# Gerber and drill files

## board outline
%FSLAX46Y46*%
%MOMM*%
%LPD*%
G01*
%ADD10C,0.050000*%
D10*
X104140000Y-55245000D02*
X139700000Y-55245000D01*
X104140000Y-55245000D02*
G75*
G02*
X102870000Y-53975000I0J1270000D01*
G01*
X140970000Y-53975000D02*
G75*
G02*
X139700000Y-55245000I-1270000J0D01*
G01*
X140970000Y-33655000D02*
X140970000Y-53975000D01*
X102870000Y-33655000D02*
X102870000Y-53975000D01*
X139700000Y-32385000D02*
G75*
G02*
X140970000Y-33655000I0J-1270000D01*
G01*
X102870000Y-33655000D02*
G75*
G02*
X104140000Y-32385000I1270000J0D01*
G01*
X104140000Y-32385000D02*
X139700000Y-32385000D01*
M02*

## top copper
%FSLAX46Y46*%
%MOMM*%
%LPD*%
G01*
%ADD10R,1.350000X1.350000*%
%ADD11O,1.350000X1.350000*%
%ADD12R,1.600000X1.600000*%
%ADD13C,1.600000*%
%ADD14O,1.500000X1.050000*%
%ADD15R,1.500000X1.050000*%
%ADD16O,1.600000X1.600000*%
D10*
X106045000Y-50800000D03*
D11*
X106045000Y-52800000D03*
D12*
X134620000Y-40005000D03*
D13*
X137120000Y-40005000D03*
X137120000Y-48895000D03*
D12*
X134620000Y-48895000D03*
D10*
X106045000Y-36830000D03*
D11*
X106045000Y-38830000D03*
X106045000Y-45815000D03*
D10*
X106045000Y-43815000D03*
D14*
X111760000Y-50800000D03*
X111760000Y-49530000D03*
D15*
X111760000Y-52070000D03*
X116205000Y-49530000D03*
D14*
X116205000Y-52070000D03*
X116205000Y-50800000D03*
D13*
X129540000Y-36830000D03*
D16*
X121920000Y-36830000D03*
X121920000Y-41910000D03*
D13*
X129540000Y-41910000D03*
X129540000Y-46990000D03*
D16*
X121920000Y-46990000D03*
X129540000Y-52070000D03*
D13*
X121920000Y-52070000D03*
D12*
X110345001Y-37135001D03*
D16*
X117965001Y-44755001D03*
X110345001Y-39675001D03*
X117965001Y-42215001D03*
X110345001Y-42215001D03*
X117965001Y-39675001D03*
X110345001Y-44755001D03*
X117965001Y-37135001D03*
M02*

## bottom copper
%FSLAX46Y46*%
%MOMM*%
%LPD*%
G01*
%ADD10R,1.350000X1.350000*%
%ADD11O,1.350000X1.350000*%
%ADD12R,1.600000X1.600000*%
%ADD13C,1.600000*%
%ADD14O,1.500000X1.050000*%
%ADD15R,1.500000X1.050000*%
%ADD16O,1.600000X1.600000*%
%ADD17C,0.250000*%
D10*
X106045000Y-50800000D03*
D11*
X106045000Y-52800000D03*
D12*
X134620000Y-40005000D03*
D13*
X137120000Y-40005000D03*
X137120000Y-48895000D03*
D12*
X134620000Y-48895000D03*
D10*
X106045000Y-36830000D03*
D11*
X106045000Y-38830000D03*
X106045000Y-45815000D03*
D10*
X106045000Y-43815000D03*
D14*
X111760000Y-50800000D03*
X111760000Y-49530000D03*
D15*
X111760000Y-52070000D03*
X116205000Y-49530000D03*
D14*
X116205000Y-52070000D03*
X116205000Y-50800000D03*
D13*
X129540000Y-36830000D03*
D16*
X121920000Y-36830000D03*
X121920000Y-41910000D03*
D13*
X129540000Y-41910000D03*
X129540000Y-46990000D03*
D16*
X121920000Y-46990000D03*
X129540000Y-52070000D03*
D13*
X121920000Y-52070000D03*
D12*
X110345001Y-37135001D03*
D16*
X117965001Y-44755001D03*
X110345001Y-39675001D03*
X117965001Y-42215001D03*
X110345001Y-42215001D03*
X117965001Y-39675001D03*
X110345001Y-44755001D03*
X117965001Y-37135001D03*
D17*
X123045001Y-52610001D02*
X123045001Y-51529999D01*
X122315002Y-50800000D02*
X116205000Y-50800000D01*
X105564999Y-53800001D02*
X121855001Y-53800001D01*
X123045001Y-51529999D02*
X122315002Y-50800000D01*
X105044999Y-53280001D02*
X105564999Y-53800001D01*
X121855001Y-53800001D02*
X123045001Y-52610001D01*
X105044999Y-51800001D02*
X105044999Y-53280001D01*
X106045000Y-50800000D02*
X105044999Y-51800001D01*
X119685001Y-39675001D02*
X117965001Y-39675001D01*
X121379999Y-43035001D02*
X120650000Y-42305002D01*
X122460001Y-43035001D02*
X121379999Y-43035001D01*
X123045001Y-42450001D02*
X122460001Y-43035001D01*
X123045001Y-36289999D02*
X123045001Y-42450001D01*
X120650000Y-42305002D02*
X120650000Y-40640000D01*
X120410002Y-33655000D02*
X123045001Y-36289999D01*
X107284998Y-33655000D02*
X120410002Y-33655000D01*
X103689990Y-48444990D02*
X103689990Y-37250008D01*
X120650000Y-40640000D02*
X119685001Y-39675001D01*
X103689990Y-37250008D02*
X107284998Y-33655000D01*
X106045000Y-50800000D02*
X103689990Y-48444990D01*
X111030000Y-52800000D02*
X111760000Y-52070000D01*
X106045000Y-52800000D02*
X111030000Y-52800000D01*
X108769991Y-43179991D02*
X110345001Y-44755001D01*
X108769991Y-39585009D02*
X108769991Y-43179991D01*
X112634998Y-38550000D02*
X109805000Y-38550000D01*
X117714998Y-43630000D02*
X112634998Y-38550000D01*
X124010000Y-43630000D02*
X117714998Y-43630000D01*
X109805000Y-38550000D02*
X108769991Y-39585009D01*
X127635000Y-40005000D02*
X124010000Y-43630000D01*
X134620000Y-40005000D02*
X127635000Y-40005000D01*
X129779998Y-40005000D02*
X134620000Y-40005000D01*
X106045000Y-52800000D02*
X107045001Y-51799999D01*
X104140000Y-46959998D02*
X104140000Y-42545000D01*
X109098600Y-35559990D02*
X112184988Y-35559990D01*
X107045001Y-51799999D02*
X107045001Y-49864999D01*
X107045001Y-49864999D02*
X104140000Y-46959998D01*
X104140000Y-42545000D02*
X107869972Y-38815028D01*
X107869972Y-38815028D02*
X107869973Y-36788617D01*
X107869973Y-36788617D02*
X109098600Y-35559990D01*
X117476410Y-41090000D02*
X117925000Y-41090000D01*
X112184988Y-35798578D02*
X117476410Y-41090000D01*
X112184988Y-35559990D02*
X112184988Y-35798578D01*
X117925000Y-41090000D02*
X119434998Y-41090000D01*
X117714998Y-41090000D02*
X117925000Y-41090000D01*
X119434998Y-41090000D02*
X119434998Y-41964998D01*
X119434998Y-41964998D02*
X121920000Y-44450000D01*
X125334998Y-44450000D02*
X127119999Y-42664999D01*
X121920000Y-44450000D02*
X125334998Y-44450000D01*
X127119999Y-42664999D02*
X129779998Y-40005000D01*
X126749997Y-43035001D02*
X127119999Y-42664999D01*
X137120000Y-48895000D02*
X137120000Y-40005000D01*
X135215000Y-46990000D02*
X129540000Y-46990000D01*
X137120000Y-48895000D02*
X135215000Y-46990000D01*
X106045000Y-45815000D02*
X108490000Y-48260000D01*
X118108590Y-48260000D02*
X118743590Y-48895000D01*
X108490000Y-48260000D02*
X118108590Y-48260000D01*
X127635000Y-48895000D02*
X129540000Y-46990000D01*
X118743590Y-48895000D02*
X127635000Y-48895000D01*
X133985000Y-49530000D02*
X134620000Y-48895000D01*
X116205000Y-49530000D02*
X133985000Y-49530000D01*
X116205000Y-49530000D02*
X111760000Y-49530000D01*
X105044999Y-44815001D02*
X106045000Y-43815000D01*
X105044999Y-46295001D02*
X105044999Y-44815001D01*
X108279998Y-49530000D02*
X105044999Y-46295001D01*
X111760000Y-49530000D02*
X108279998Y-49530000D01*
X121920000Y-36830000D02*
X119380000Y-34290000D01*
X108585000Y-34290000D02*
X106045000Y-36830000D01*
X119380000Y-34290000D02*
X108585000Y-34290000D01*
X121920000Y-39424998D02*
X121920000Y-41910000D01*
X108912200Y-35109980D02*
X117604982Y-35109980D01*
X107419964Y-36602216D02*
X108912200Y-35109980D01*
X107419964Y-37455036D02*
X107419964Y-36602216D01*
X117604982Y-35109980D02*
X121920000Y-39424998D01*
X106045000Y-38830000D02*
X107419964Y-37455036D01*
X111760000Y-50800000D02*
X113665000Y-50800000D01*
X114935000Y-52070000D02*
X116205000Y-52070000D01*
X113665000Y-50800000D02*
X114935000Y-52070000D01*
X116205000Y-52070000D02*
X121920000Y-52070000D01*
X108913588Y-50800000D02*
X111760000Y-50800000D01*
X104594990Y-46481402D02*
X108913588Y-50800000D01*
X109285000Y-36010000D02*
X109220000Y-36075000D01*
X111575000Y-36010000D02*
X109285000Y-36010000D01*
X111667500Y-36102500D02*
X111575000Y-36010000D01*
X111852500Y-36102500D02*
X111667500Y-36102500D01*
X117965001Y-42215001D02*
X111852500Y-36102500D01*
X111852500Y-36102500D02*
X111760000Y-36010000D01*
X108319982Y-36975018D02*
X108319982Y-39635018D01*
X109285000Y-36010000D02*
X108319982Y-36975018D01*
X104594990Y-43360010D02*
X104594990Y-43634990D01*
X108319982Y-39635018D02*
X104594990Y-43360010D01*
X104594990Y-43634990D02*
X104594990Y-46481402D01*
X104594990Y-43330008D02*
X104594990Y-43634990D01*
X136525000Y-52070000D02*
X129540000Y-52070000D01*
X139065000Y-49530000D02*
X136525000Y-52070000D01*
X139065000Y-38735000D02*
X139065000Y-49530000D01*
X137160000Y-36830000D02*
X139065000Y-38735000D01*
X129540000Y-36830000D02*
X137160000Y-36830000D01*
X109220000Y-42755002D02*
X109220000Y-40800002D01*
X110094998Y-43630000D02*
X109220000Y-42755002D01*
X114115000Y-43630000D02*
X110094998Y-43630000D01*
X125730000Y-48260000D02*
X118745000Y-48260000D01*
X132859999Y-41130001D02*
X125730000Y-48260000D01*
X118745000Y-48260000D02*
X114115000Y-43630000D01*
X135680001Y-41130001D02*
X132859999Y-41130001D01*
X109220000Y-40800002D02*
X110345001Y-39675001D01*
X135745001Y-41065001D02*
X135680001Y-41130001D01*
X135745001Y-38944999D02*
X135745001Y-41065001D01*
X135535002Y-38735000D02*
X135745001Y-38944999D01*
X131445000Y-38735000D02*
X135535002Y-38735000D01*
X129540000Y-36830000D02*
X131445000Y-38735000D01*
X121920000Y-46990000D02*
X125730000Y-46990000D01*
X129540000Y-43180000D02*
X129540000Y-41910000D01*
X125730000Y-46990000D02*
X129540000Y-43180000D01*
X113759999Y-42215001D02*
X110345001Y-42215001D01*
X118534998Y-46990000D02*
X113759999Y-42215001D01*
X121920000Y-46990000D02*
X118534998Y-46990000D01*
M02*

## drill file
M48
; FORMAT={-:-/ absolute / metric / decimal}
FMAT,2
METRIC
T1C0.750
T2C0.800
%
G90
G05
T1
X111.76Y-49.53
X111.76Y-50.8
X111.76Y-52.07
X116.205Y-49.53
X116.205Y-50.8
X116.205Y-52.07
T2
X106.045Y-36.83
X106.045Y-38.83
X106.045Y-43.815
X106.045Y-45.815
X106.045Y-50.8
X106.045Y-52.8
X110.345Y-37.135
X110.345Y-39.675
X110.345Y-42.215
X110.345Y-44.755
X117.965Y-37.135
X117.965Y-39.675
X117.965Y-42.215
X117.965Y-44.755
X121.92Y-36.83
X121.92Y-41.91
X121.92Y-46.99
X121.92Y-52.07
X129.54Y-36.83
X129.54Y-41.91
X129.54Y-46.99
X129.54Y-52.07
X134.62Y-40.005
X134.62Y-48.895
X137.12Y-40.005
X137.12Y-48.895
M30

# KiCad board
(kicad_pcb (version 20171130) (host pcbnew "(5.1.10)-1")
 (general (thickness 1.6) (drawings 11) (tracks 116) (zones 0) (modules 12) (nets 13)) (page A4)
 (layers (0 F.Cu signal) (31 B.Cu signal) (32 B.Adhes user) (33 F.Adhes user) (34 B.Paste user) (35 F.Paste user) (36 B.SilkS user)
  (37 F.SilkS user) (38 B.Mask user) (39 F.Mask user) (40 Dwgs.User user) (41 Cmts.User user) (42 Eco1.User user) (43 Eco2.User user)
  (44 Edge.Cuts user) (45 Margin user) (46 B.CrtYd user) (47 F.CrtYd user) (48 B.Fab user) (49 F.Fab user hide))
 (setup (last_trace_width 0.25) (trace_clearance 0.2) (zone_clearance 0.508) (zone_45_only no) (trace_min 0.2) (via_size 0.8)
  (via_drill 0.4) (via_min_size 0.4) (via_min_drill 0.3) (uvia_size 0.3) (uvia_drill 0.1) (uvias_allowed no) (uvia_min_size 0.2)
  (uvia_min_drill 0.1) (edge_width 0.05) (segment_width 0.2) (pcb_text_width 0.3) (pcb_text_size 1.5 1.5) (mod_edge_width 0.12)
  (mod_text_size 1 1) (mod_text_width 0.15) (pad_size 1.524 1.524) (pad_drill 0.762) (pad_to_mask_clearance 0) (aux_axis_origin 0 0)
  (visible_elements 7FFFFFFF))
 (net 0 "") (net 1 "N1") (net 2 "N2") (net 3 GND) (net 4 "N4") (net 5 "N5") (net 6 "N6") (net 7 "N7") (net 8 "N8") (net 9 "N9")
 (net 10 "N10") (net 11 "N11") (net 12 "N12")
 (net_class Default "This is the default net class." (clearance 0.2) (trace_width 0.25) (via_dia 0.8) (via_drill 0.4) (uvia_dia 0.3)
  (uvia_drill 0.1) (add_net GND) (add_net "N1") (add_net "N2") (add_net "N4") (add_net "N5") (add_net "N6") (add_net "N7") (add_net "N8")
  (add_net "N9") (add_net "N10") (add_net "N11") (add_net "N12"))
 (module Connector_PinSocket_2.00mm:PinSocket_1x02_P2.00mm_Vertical (layer F.Cu) (at 106.045 50.8)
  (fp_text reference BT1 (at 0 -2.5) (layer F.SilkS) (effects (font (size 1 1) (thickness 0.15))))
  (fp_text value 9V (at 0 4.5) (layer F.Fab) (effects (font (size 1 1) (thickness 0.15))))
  (pad 1 thru_hole rect (at 0 0) (size 1.35 1.35) (drill 0.8) (layers *.Cu *.Mask) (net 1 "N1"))
  (pad 2 thru_hole oval (at 0 2) (size 1.35 1.35) (drill 0.8) (layers *.Cu *.Mask) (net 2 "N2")))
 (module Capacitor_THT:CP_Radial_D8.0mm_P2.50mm (layer F.Cu) (at 134.62 40.005)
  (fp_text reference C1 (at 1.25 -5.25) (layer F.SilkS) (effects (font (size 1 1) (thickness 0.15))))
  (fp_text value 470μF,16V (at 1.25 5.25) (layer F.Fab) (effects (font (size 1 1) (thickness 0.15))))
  (pad 1 thru_hole rect (at 0 0) (size 1.6 1.6) (drill 0.8) (layers *.Cu *.Mask) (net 2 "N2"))
  (pad 2 thru_hole circle (at 2.5 0) (size 1.6 1.6) (drill 0.8) (layers *.Cu *.Mask) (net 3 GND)))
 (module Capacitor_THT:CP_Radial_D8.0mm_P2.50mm (layer F.Cu) (at 134.62 48.895)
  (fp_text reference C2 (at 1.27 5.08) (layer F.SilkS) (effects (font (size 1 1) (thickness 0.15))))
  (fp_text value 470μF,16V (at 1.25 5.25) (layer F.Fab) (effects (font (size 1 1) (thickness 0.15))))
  (pad 2 thru_hole circle (at 2.5 0) (size 1.6 1.6) (drill 0.8) (layers *.Cu *.Mask) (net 3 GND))
  (pad 1 thru_hole rect (at 0 0) (size 1.6 1.6) (drill 0.8) (layers *.Cu *.Mask) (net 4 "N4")))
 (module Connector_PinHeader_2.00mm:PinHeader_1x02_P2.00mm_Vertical (layer F.Cu) (at 106.045 36.83)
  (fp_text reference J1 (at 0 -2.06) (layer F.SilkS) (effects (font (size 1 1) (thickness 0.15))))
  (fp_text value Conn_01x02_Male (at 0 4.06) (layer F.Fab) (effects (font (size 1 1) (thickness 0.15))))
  (pad 1 thru_hole rect (at 0 0) (size 1.35 1.35) (drill 0.8) (layers *.Cu *.Mask) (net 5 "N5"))
  (pad 2 thru_hole oval (at 0 2) (size 1.35 1.35) (drill 0.8) (layers *.Cu *.Mask) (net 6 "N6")))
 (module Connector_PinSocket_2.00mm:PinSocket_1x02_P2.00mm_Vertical (layer F.Cu) (at 106.045 43.815)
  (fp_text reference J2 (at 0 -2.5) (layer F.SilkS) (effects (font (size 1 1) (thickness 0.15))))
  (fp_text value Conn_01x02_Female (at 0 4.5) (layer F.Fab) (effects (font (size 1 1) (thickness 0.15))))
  (pad 2 thru_hole oval (at 0 2) (size 1.35 1.35) (drill 0.8) (layers *.Cu *.Mask) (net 3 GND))
  (pad 1 thru_hole rect (at 0 0) (size 1.35 1.35) (drill 0.8) (layers *.Cu *.Mask) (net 4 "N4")))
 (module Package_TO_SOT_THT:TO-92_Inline (layer F.Cu) (at 111.76 52.07 90)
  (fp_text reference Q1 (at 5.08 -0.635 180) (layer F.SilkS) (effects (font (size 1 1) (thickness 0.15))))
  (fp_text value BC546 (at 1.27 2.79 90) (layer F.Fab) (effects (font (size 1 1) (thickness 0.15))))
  (pad 2 thru_hole oval (at 1.27 0 90) (size 1.05 1.5) (drill 0.75) (layers *.Cu *.Mask) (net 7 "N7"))
  (pad 3 thru_hole oval (at 2.54 0 90) (size 1.05 1.5) (drill 0.75) (layers *.Cu *.Mask) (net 4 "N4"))
  (pad 1 thru_hole rect (at 0 0 90) (size 1.05 1.5) (drill 0.75) (layers *.Cu *.Mask) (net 2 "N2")))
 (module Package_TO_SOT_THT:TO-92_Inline (layer F.Cu) (at 116.205 49.53 270)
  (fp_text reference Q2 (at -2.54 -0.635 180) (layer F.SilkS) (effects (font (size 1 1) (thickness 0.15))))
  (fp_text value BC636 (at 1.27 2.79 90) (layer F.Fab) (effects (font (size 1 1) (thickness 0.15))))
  (pad 1 thru_hole rect (at 0 0 270) (size 1.05 1.5) (drill 0.75) (layers *.Cu *.Mask) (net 4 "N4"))
  (pad 3 thru_hole oval (at 2.54 0 270) (size 1.05 1.5) (drill 0.75) (layers *.Cu *.Mask) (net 7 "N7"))
  (pad 2 thru_hole oval (at 1.27 0 270) (size 1.05 1.5) (drill 0.75) (layers *.Cu *.Mask) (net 1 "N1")))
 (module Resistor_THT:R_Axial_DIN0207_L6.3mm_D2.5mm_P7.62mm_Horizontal (layer F.Cu) (at 129.54 36.83 180)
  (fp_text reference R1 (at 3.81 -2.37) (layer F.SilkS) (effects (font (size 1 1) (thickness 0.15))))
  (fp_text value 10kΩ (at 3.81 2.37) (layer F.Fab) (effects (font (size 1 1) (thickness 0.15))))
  (pad 1 thru_hole circle (at 0 0 180) (size 1.6 1.6) (drill 0.8) (layers *.Cu *.Mask) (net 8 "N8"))
  (pad 2 thru_hole oval (at 7.62 0 180) (size 1.6 1.6) (drill 0.8) (layers *.Cu *.Mask) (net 5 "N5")))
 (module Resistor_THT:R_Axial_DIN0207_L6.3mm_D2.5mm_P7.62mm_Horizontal (layer F.Cu) (at 129.54 41.91 180)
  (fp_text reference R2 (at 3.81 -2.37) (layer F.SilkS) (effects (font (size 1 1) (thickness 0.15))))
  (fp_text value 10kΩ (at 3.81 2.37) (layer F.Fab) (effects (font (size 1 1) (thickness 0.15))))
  (pad 2 thru_hole oval (at 7.62 0 180) (size 1.6 1.6) (drill 0.8) (layers *.Cu *.Mask) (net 6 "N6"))
  (pad 1 thru_hole circle (at 0 0 180) (size 1.6 1.6) (drill 0.8) (layers *.Cu *.Mask) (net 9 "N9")))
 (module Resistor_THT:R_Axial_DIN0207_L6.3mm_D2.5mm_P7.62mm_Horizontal (layer F.Cu) (at 129.54 46.99 180)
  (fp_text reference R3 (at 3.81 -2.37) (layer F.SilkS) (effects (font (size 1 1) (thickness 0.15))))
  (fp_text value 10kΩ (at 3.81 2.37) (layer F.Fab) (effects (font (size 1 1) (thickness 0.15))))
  (pad 1 thru_hole circle (at 0 0 180) (size 1.6 1.6) (drill 0.8) (layers *.Cu *.Mask) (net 3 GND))
  (pad 2 thru_hole oval (at 7.62 0 180) (size 1.6 1.6) (drill 0.8) (layers *.Cu *.Mask) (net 9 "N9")))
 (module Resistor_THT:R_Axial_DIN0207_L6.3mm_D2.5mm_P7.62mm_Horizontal (layer F.Cu) (at 121.92 52.07)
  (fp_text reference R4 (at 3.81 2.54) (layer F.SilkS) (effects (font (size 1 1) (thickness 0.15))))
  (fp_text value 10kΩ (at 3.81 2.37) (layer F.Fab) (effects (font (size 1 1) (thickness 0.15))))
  (pad 2 thru_hole oval (at 7.62 0) (size 1.6 1.6) (drill 0.8) (layers *.Cu *.Mask) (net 8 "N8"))
  (pad 1 thru_hole circle (at 0 0) (size 1.6 1.6) (drill 0.8) (layers *.Cu *.Mask) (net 7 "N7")))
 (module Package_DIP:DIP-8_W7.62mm (layer F.Cu) (at 110.345001 37.135001)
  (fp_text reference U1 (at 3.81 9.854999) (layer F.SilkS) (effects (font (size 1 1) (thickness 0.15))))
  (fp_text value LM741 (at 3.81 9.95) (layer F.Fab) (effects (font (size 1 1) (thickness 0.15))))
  (pad 1 thru_hole rect (at 0 0) (size 1.6 1.6) (drill 0.8) (layers *.Cu *.Mask) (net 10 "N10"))
  (pad 5 thru_hole oval (at 7.62 7.62) (size 1.6 1.6) (drill 0.8) (layers *.Cu *.Mask) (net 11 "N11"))
  (pad 2 thru_hole oval (at 0 2.54) (size 1.6 1.6) (drill 0.8) (layers *.Cu *.Mask) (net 8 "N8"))
  (pad 6 thru_hole oval (at 7.62 5.08) (size 1.6 1.6) (drill 0.8) (layers *.Cu *.Mask) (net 7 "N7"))
  (pad 3 thru_hole oval (at 0 5.08) (size 1.6 1.6) (drill 0.8) (layers *.Cu *.Mask) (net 9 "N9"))
  (pad 7 thru_hole oval (at 7.62 2.54) (size 1.6 1.6) (drill 0.8) (layers *.Cu *.Mask) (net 1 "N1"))
  (pad 4 thru_hole oval (at 0 7.62) (size 1.6 1.6) (drill 0.8) (layers *.Cu *.Mask) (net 2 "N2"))
  (pad 8 thru_hole oval (at 7.62 0) (size 1.6 1.6) (drill 0.8) (layers *.Cu *.Mask) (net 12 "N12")))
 (gr_line (start 104.14 55.245) (end 139.7 55.245) (layer Edge.Cuts) (width 0.05))
 (gr_arc (start 104.14 53.975) (end 102.87 53.975) (angle -90) (layer Edge.Cuts) (width 0.05))
 (gr_arc (start 139.7 53.975) (end 139.7 55.245) (angle -90) (layer Edge.Cuts) (width 0.05))
 (gr_line (start 140.97 33.655) (end 140.97 53.975) (layer Edge.Cuts) (width 0.05))
 (gr_line (start 102.87 33.655) (end 102.87 53.975) (layer Edge.Cuts) (width 0.05))
 (gr_arc (start 139.7 33.655) (end 140.97 33.655) (angle -90) (layer Edge.Cuts) (width 0.05))
 (gr_arc (start 104.14 33.655) (end 104.14 32.385) (angle -90) (layer Edge.Cuts) (width 0.05))
 (gr_line (start 104.14 32.385) (end 139.7 32.385) (layer Edge.Cuts) (width 0.05))
 (segment (start 123.045001 52.610001) (end 123.045001 51.529999) (width 0.25) (layer B.Cu) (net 1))
 (segment (start 122.315002 50.8) (end 116.205 50.8) (width 0.25) (layer B.Cu) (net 1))
 (segment (start 105.564999 53.800001) (end 121.855001 53.800001) (width 0.25) (layer B.Cu) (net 1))
 (segment (start 123.045001 51.529999) (end 122.315002 50.8) (width 0.25) (layer B.Cu) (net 1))
 (segment (start 105.044999 53.280001) (end 105.564999 53.800001) (width 0.25) (layer B.Cu) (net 1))
 (segment (start 121.855001 53.800001) (end 123.045001 52.610001) (width 0.25) (layer B.Cu) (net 1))
 (segment (start 105.044999 51.800001) (end 105.044999 53.280001) (width 0.25) (layer B.Cu) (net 1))
 (segment (start 106.045 50.8) (end 105.044999 51.800001) (width 0.25) (layer B.Cu) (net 1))
 (segment (start 119.685001 39.675001) (end 117.965001 39.675001) (width 0.25) (layer B.Cu) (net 1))
 (segment (start 121.379999 43.035001) (end 120.65 42.305002) (width 0.25) (layer B.Cu) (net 1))
 (segment (start 122.460001 43.035001) (end 121.379999 43.035001) (width 0.25) (layer B.Cu) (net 1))
 (segment (start 123.045001 42.450001) (end 122.460001 43.035001) (width 0.25) (layer B.Cu) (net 1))
 (segment (start 123.045001 36.289999) (end 123.045001 42.450001) (width 0.25) (layer B.Cu) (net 1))
 (segment (start 120.65 42.305002) (end 120.65 40.64) (width 0.25) (layer B.Cu) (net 1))
 (segment (start 120.410002 33.655) (end 123.045001 36.289999) (width 0.25) (layer B.Cu) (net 1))
 (segment (start 107.284998 33.655) (end 120.410002 33.655) (width 0.25) (layer B.Cu) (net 1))
 (segment (start 103.68999 48.44499) (end 103.68999 37.250008) (width 0.25) (layer B.Cu) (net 1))
 (segment (start 120.65 40.64) (end 119.685001 39.675001) (width 0.25) (layer B.Cu) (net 1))
 (segment (start 103.68999 37.250008) (end 107.284998 33.655) (width 0.25) (layer B.Cu) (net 1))
 (segment (start 106.045 50.8) (end 103.68999 48.44499) (width 0.25) (layer B.Cu) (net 1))
 (segment (start 111.03 52.8) (end 111.76 52.07) (width 0.25) (layer B.Cu) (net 2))
 (segment (start 106.045 52.8) (end 111.03 52.8) (width 0.25) (layer B.Cu) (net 2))
 (segment (start 108.769991 43.179991) (end 110.345001 44.755001) (width 0.25) (layer B.Cu) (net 2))
 (segment (start 108.769991 39.585009) (end 108.769991 43.179991) (width 0.25) (layer B.Cu) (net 2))
 (segment (start 112.634998 38.55) (end 109.805 38.55) (width 0.25) (layer B.Cu) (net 2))
 (segment (start 117.714998 43.63) (end 112.634998 38.55) (width 0.25) (layer B.Cu) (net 2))
 (segment (start 124.01 43.63) (end 117.714998 43.63) (width 0.25) (layer B.Cu) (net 2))
 (segment (start 109.805 38.55) (end 108.769991 39.585009) (width 0.25) (layer B.Cu) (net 2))
 (segment (start 127.635 40.005) (end 124.01 43.63) (width 0.25) (layer B.Cu) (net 2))
 (segment (start 134.62 40.005) (end 127.635 40.005) (width 0.25) (layer B.Cu) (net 2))
 (segment (start 129.779998 40.005) (end 134.62 40.005) (width 0.25) (layer B.Cu) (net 2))
 (segment (start 106.045 52.8) (end 107.045001 51.799999) (width 0.25) (layer B.Cu) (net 2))
 (segment (start 104.14 46.959998) (end 104.14 42.545) (width 0.25) (layer B.Cu) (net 2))
 (segment (start 109.0986 35.55999) (end 112.184988 35.55999) (width 0.25) (layer B.Cu) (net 2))
 (segment (start 107.045001 51.799999) (end 107.045001 49.864999) (width 0.25) (layer B.Cu) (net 2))
 (segment (start 107.045001 49.864999) (end 104.14 46.959998) (width 0.25) (layer B.Cu) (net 2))
 (segment (start 104.14 42.545) (end 107.869972 38.815028) (width 0.25) (layer B.Cu) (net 2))
 (segment (start 107.869972 38.815028) (end 107.869973 36.788617) (width 0.25) (layer B.Cu) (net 2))
 (segment (start 107.869973 36.788617) (end 109.0986 35.55999) (width 0.25) (layer B.Cu) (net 2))
 (segment (start 117.47641 41.09) (end 117.925 41.09) (width 0.25) (layer B.Cu) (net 2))
 (segment (start 112.184988 35.798578) (end 117.47641 41.09) (width 0.25) (layer B.Cu) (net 2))
 (segment (start 112.184988 35.55999) (end 112.184988 35.798578) (width 0.25) (layer B.Cu) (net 2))
 (segment (start 117.925 41.09) (end 119.434998 41.09) (width 0.25) (layer B.Cu) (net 2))
 (segment (start 117.714998 41.09) (end 117.925 41.09) (width 0.25) (layer B.Cu) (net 2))
 (segment (start 119.434998 41.09) (end 119.434998 41.964998) (width 0.25) (layer B.Cu) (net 2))
 (segment (start 119.434998 41.964998) (end 121.92 44.45) (width 0.25) (layer B.Cu) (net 2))
 (segment (start 125.334998 44.45) (end 127.119999 42.664999) (width 0.25) (layer B.Cu) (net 2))
 (segment (start 121.92 44.45) (end 125.334998 44.45) (width 0.25) (layer B.Cu) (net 2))
 (segment (start 127.119999 42.664999) (end 129.779998 40.005) (width 0.25) (layer B.Cu) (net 2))
 (segment (start 126.749997 43.035001) (end 127.119999 42.664999) (width 0.25) (layer B.Cu) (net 2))
 (segment (start 137.12 48.895) (end 137.12 40.005) (width 0.25) (layer B.Cu) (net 3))
 (segment (start 135.215 46.99) (end 129.54 46.99) (width 0.25) (layer B.Cu) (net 3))
 (segment (start 137.12 48.895) (end 135.215 46.99) (width 0.25) (layer B.Cu) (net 3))
 (segment (start 106.045 45.815) (end 108.49 48.26) (width 0.25) (layer B.Cu) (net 3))
 (segment (start 118.10859 48.26) (end 118.74359 48.895) (width 0.25) (layer B.Cu) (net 3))
 (segment (start 108.49 48.26) (end 118.10859 48.26) (width 0.25) (layer B.Cu) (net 3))
 (segment (start 127.635 48.895) (end 129.54 46.99) (width 0.25) (layer B.Cu) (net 3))
 (segment (start 118.74359 48.895) (end 127.635 48.895) (width 0.25) (layer B.Cu) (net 3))
 (segment (start 133.985 49.53) (end 134.62 48.895) (width 0.25) (layer B.Cu) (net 4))
 (segment (start 116.205 49.53) (end 133.985 49.53) (width 0.25) (layer B.Cu) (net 4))
 (segment (start 116.205 49.53) (end 111.76 49.53) (width 0.25) (layer B.Cu) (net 4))
 (segment (start 105.044999 44.815001) (end 106.045 43.815) (width 0.25) (layer B.Cu) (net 4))
 (segment (start 105.044999 46.295001) (end 105.044999 44.815001) (width 0.25) (layer B.Cu) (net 4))
 (segment (start 108.279998 49.53) (end 105.044999 46.295001) (width 0.25) (layer B.Cu) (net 4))
 (segment (start 111.76 49.53) (end 108.279998 49.53) (width 0.25) (layer B.Cu) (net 4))
 (segment (start 121.92 36.83) (end 119.38 34.29) (width 0.25) (layer B.Cu) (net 5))
 (segment (start 108.585 34.29) (end 106.045 36.83) (width 0.25) (layer B.Cu) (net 5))
 (segment (start 119.38 34.29) (end 108.585 34.29) (width 0.25) (layer B.Cu) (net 5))
 (segment (start 121.92 39.424998) (end 121.92 41.91) (width 0.25) (layer B.Cu) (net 6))
 (segment (start 108.9122 35.10998) (end 117.604982 35.10998) (width 0.25) (layer B.Cu) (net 6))
 (segment (start 107.419964 36.602216) (end 108.9122 35.10998) (width 0.25) (layer B.Cu) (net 6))
 (segment (start 107.419964 37.455036) (end 107.419964 36.602216) (width 0.25) (layer B.Cu) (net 6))
 (segment (start 117.604982 35.10998) (end 121.92 39.424998) (width 0.25) (layer B.Cu) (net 6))
 (segment (start 106.045 38.83) (end 107.419964 37.455036) (width 0.25) (layer B.Cu) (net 6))
 (segment (start 111.76 50.8) (end 113.665 50.8) (width 0.25) (layer B.Cu) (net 7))
 (segment (start 114.935 52.07) (end 116.205 52.07) (width 0.25) (layer B.Cu) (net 7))
 (segment (start 113.665 50.8) (end 114.935 52.07) (width 0.25) (layer B.Cu) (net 7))
 (segment (start 116.205 52.07) (end 121.92 52.07) (width 0.25) (layer B.Cu) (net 7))
 (segment (start 108.913588 50.8) (end 111.76 50.8) (width 0.25) (layer B.Cu) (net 7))
 (segment (start 104.59499 46.481402) (end 108.913588 50.8) (width 0.25) (layer B.Cu) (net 7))
 (segment (start 109.285 36.01) (end 109.22 36.075) (width 0.25) (layer B.Cu) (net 7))
 (segment (start 111.575 36.01) (end 109.285 36.01) (width 0.25) (layer B.Cu) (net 7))
 (segment (start 111.6675 36.1025) (end 111.575 36.01) (width 0.25) (layer B.Cu) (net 7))
 (segment (start 111.8525 36.1025) (end 111.6675 36.1025) (width 0.25) (layer B.Cu) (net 7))
 (segment (start 117.965001 42.215001) (end 111.8525 36.1025) (width 0.25) (layer B.Cu) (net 7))
 (segment (start 111.8525 36.1025) (end 111.76 36.01) (width 0.25) (layer B.Cu) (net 7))
 (segment (start 108.319982 36.975018) (end 108.319982 39.635018) (width 0.25) (layer B.Cu) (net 7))
 (segment (start 109.285 36.01) (end 108.319982 36.975018) (width 0.25) (layer B.Cu) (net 7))
 (segment (start 104.59499 43.36001) (end 104.59499 43.63499) (width 0.25) (layer B.Cu) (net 7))
 (segment (start 108.319982 39.635018) (end 104.59499 43.36001) (width 0.25) (layer B.Cu) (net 7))
 (segment (start 104.59499 43.63499) (end 104.59499 46.481402) (width 0.25) (layer B.Cu) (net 7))
 (segment (start 104.59499 43.330008) (end 104.59499 43.63499) (width 0.25) (layer B.Cu) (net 7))
 (segment (start 136.525 52.07) (end 129.54 52.07) (width 0.25) (layer B.Cu) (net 8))
 (segment (start 139.065 49.53) (end 136.525 52.07) (width 0.25) (layer B.Cu) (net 8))
 (segment (start 139.065 38.735) (end 139.065 49.53) (width 0.25) (layer B.Cu) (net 8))
 (segment (start 137.16 36.83) (end 139.065 38.735) (width 0.25) (layer B.Cu) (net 8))
 (segment (start 129.54 36.83) (end 137.16 36.83) (width 0.25) (layer B.Cu) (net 8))
 (segment (start 109.22 42.755002) (end 109.22 40.800002) (width 0.25) (layer B.Cu) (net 8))
 (segment (start 110.094998 43.63) (end 109.22 42.755002) (width 0.25) (layer B.Cu) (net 8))
 (segment (start 114.115 43.63) (end 110.094998 43.63) (width 0.25) (layer B.Cu) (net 8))
 (segment (start 125.73 48.26) (end 118.745 48.26) (width 0.25) (layer B.Cu) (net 8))
 (segment (start 132.859999 41.130001) (end 125.73 48.26) (width 0.25) (layer B.Cu) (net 8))
 (segment (start 118.745 48.26) (end 114.115 43.63) (width 0.25) (layer B.Cu) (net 8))
 (segment (start 135.680001 41.130001) (end 132.859999 41.130001) (width 0.25) (layer B.Cu) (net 8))
 (segment (start 109.22 40.800002) (end 110.345001 39.675001) (width 0.25) (layer B.Cu) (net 8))
 (segment (start 135.745001 41.065001) (end 135.680001 41.130001) (width 0.25) (layer B.Cu) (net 8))
 (segment (start 135.745001 38.944999) (end 135.745001 41.065001) (width 0.25) (layer B.Cu) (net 8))
 (segment (start 135.535002 38.735) (end 135.745001 38.944999) (width 0.25) (layer B.Cu) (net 8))
 (segment (start 131.445 38.735) (end 135.535002 38.735) (width 0.25) (layer B.Cu) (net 8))
 (segment (start 129.54 36.83) (end 131.445 38.735) (width 0.25) (layer B.Cu) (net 8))
 (segment (start 121.92 46.99) (end 125.73 46.99) (width 0.25) (layer B.Cu) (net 9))
 (segment (start 129.54 43.18) (end 129.54 41.91) (width 0.25) (layer B.Cu) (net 9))
 (segment (start 125.73 46.99) (end 129.54 43.18) (width 0.25) (layer B.Cu) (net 9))
 (segment (start 113.759999 42.215001) (end 110.345001 42.215001) (width 0.25) (layer B.Cu) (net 9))
 (segment (start 118.534998 46.99) (end 113.759999 42.215001) (width 0.25) (layer B.Cu) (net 9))
 (segment (start 121.92 46.99) (end 118.534998 46.99) (width 0.25) (layer B.Cu) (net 9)))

